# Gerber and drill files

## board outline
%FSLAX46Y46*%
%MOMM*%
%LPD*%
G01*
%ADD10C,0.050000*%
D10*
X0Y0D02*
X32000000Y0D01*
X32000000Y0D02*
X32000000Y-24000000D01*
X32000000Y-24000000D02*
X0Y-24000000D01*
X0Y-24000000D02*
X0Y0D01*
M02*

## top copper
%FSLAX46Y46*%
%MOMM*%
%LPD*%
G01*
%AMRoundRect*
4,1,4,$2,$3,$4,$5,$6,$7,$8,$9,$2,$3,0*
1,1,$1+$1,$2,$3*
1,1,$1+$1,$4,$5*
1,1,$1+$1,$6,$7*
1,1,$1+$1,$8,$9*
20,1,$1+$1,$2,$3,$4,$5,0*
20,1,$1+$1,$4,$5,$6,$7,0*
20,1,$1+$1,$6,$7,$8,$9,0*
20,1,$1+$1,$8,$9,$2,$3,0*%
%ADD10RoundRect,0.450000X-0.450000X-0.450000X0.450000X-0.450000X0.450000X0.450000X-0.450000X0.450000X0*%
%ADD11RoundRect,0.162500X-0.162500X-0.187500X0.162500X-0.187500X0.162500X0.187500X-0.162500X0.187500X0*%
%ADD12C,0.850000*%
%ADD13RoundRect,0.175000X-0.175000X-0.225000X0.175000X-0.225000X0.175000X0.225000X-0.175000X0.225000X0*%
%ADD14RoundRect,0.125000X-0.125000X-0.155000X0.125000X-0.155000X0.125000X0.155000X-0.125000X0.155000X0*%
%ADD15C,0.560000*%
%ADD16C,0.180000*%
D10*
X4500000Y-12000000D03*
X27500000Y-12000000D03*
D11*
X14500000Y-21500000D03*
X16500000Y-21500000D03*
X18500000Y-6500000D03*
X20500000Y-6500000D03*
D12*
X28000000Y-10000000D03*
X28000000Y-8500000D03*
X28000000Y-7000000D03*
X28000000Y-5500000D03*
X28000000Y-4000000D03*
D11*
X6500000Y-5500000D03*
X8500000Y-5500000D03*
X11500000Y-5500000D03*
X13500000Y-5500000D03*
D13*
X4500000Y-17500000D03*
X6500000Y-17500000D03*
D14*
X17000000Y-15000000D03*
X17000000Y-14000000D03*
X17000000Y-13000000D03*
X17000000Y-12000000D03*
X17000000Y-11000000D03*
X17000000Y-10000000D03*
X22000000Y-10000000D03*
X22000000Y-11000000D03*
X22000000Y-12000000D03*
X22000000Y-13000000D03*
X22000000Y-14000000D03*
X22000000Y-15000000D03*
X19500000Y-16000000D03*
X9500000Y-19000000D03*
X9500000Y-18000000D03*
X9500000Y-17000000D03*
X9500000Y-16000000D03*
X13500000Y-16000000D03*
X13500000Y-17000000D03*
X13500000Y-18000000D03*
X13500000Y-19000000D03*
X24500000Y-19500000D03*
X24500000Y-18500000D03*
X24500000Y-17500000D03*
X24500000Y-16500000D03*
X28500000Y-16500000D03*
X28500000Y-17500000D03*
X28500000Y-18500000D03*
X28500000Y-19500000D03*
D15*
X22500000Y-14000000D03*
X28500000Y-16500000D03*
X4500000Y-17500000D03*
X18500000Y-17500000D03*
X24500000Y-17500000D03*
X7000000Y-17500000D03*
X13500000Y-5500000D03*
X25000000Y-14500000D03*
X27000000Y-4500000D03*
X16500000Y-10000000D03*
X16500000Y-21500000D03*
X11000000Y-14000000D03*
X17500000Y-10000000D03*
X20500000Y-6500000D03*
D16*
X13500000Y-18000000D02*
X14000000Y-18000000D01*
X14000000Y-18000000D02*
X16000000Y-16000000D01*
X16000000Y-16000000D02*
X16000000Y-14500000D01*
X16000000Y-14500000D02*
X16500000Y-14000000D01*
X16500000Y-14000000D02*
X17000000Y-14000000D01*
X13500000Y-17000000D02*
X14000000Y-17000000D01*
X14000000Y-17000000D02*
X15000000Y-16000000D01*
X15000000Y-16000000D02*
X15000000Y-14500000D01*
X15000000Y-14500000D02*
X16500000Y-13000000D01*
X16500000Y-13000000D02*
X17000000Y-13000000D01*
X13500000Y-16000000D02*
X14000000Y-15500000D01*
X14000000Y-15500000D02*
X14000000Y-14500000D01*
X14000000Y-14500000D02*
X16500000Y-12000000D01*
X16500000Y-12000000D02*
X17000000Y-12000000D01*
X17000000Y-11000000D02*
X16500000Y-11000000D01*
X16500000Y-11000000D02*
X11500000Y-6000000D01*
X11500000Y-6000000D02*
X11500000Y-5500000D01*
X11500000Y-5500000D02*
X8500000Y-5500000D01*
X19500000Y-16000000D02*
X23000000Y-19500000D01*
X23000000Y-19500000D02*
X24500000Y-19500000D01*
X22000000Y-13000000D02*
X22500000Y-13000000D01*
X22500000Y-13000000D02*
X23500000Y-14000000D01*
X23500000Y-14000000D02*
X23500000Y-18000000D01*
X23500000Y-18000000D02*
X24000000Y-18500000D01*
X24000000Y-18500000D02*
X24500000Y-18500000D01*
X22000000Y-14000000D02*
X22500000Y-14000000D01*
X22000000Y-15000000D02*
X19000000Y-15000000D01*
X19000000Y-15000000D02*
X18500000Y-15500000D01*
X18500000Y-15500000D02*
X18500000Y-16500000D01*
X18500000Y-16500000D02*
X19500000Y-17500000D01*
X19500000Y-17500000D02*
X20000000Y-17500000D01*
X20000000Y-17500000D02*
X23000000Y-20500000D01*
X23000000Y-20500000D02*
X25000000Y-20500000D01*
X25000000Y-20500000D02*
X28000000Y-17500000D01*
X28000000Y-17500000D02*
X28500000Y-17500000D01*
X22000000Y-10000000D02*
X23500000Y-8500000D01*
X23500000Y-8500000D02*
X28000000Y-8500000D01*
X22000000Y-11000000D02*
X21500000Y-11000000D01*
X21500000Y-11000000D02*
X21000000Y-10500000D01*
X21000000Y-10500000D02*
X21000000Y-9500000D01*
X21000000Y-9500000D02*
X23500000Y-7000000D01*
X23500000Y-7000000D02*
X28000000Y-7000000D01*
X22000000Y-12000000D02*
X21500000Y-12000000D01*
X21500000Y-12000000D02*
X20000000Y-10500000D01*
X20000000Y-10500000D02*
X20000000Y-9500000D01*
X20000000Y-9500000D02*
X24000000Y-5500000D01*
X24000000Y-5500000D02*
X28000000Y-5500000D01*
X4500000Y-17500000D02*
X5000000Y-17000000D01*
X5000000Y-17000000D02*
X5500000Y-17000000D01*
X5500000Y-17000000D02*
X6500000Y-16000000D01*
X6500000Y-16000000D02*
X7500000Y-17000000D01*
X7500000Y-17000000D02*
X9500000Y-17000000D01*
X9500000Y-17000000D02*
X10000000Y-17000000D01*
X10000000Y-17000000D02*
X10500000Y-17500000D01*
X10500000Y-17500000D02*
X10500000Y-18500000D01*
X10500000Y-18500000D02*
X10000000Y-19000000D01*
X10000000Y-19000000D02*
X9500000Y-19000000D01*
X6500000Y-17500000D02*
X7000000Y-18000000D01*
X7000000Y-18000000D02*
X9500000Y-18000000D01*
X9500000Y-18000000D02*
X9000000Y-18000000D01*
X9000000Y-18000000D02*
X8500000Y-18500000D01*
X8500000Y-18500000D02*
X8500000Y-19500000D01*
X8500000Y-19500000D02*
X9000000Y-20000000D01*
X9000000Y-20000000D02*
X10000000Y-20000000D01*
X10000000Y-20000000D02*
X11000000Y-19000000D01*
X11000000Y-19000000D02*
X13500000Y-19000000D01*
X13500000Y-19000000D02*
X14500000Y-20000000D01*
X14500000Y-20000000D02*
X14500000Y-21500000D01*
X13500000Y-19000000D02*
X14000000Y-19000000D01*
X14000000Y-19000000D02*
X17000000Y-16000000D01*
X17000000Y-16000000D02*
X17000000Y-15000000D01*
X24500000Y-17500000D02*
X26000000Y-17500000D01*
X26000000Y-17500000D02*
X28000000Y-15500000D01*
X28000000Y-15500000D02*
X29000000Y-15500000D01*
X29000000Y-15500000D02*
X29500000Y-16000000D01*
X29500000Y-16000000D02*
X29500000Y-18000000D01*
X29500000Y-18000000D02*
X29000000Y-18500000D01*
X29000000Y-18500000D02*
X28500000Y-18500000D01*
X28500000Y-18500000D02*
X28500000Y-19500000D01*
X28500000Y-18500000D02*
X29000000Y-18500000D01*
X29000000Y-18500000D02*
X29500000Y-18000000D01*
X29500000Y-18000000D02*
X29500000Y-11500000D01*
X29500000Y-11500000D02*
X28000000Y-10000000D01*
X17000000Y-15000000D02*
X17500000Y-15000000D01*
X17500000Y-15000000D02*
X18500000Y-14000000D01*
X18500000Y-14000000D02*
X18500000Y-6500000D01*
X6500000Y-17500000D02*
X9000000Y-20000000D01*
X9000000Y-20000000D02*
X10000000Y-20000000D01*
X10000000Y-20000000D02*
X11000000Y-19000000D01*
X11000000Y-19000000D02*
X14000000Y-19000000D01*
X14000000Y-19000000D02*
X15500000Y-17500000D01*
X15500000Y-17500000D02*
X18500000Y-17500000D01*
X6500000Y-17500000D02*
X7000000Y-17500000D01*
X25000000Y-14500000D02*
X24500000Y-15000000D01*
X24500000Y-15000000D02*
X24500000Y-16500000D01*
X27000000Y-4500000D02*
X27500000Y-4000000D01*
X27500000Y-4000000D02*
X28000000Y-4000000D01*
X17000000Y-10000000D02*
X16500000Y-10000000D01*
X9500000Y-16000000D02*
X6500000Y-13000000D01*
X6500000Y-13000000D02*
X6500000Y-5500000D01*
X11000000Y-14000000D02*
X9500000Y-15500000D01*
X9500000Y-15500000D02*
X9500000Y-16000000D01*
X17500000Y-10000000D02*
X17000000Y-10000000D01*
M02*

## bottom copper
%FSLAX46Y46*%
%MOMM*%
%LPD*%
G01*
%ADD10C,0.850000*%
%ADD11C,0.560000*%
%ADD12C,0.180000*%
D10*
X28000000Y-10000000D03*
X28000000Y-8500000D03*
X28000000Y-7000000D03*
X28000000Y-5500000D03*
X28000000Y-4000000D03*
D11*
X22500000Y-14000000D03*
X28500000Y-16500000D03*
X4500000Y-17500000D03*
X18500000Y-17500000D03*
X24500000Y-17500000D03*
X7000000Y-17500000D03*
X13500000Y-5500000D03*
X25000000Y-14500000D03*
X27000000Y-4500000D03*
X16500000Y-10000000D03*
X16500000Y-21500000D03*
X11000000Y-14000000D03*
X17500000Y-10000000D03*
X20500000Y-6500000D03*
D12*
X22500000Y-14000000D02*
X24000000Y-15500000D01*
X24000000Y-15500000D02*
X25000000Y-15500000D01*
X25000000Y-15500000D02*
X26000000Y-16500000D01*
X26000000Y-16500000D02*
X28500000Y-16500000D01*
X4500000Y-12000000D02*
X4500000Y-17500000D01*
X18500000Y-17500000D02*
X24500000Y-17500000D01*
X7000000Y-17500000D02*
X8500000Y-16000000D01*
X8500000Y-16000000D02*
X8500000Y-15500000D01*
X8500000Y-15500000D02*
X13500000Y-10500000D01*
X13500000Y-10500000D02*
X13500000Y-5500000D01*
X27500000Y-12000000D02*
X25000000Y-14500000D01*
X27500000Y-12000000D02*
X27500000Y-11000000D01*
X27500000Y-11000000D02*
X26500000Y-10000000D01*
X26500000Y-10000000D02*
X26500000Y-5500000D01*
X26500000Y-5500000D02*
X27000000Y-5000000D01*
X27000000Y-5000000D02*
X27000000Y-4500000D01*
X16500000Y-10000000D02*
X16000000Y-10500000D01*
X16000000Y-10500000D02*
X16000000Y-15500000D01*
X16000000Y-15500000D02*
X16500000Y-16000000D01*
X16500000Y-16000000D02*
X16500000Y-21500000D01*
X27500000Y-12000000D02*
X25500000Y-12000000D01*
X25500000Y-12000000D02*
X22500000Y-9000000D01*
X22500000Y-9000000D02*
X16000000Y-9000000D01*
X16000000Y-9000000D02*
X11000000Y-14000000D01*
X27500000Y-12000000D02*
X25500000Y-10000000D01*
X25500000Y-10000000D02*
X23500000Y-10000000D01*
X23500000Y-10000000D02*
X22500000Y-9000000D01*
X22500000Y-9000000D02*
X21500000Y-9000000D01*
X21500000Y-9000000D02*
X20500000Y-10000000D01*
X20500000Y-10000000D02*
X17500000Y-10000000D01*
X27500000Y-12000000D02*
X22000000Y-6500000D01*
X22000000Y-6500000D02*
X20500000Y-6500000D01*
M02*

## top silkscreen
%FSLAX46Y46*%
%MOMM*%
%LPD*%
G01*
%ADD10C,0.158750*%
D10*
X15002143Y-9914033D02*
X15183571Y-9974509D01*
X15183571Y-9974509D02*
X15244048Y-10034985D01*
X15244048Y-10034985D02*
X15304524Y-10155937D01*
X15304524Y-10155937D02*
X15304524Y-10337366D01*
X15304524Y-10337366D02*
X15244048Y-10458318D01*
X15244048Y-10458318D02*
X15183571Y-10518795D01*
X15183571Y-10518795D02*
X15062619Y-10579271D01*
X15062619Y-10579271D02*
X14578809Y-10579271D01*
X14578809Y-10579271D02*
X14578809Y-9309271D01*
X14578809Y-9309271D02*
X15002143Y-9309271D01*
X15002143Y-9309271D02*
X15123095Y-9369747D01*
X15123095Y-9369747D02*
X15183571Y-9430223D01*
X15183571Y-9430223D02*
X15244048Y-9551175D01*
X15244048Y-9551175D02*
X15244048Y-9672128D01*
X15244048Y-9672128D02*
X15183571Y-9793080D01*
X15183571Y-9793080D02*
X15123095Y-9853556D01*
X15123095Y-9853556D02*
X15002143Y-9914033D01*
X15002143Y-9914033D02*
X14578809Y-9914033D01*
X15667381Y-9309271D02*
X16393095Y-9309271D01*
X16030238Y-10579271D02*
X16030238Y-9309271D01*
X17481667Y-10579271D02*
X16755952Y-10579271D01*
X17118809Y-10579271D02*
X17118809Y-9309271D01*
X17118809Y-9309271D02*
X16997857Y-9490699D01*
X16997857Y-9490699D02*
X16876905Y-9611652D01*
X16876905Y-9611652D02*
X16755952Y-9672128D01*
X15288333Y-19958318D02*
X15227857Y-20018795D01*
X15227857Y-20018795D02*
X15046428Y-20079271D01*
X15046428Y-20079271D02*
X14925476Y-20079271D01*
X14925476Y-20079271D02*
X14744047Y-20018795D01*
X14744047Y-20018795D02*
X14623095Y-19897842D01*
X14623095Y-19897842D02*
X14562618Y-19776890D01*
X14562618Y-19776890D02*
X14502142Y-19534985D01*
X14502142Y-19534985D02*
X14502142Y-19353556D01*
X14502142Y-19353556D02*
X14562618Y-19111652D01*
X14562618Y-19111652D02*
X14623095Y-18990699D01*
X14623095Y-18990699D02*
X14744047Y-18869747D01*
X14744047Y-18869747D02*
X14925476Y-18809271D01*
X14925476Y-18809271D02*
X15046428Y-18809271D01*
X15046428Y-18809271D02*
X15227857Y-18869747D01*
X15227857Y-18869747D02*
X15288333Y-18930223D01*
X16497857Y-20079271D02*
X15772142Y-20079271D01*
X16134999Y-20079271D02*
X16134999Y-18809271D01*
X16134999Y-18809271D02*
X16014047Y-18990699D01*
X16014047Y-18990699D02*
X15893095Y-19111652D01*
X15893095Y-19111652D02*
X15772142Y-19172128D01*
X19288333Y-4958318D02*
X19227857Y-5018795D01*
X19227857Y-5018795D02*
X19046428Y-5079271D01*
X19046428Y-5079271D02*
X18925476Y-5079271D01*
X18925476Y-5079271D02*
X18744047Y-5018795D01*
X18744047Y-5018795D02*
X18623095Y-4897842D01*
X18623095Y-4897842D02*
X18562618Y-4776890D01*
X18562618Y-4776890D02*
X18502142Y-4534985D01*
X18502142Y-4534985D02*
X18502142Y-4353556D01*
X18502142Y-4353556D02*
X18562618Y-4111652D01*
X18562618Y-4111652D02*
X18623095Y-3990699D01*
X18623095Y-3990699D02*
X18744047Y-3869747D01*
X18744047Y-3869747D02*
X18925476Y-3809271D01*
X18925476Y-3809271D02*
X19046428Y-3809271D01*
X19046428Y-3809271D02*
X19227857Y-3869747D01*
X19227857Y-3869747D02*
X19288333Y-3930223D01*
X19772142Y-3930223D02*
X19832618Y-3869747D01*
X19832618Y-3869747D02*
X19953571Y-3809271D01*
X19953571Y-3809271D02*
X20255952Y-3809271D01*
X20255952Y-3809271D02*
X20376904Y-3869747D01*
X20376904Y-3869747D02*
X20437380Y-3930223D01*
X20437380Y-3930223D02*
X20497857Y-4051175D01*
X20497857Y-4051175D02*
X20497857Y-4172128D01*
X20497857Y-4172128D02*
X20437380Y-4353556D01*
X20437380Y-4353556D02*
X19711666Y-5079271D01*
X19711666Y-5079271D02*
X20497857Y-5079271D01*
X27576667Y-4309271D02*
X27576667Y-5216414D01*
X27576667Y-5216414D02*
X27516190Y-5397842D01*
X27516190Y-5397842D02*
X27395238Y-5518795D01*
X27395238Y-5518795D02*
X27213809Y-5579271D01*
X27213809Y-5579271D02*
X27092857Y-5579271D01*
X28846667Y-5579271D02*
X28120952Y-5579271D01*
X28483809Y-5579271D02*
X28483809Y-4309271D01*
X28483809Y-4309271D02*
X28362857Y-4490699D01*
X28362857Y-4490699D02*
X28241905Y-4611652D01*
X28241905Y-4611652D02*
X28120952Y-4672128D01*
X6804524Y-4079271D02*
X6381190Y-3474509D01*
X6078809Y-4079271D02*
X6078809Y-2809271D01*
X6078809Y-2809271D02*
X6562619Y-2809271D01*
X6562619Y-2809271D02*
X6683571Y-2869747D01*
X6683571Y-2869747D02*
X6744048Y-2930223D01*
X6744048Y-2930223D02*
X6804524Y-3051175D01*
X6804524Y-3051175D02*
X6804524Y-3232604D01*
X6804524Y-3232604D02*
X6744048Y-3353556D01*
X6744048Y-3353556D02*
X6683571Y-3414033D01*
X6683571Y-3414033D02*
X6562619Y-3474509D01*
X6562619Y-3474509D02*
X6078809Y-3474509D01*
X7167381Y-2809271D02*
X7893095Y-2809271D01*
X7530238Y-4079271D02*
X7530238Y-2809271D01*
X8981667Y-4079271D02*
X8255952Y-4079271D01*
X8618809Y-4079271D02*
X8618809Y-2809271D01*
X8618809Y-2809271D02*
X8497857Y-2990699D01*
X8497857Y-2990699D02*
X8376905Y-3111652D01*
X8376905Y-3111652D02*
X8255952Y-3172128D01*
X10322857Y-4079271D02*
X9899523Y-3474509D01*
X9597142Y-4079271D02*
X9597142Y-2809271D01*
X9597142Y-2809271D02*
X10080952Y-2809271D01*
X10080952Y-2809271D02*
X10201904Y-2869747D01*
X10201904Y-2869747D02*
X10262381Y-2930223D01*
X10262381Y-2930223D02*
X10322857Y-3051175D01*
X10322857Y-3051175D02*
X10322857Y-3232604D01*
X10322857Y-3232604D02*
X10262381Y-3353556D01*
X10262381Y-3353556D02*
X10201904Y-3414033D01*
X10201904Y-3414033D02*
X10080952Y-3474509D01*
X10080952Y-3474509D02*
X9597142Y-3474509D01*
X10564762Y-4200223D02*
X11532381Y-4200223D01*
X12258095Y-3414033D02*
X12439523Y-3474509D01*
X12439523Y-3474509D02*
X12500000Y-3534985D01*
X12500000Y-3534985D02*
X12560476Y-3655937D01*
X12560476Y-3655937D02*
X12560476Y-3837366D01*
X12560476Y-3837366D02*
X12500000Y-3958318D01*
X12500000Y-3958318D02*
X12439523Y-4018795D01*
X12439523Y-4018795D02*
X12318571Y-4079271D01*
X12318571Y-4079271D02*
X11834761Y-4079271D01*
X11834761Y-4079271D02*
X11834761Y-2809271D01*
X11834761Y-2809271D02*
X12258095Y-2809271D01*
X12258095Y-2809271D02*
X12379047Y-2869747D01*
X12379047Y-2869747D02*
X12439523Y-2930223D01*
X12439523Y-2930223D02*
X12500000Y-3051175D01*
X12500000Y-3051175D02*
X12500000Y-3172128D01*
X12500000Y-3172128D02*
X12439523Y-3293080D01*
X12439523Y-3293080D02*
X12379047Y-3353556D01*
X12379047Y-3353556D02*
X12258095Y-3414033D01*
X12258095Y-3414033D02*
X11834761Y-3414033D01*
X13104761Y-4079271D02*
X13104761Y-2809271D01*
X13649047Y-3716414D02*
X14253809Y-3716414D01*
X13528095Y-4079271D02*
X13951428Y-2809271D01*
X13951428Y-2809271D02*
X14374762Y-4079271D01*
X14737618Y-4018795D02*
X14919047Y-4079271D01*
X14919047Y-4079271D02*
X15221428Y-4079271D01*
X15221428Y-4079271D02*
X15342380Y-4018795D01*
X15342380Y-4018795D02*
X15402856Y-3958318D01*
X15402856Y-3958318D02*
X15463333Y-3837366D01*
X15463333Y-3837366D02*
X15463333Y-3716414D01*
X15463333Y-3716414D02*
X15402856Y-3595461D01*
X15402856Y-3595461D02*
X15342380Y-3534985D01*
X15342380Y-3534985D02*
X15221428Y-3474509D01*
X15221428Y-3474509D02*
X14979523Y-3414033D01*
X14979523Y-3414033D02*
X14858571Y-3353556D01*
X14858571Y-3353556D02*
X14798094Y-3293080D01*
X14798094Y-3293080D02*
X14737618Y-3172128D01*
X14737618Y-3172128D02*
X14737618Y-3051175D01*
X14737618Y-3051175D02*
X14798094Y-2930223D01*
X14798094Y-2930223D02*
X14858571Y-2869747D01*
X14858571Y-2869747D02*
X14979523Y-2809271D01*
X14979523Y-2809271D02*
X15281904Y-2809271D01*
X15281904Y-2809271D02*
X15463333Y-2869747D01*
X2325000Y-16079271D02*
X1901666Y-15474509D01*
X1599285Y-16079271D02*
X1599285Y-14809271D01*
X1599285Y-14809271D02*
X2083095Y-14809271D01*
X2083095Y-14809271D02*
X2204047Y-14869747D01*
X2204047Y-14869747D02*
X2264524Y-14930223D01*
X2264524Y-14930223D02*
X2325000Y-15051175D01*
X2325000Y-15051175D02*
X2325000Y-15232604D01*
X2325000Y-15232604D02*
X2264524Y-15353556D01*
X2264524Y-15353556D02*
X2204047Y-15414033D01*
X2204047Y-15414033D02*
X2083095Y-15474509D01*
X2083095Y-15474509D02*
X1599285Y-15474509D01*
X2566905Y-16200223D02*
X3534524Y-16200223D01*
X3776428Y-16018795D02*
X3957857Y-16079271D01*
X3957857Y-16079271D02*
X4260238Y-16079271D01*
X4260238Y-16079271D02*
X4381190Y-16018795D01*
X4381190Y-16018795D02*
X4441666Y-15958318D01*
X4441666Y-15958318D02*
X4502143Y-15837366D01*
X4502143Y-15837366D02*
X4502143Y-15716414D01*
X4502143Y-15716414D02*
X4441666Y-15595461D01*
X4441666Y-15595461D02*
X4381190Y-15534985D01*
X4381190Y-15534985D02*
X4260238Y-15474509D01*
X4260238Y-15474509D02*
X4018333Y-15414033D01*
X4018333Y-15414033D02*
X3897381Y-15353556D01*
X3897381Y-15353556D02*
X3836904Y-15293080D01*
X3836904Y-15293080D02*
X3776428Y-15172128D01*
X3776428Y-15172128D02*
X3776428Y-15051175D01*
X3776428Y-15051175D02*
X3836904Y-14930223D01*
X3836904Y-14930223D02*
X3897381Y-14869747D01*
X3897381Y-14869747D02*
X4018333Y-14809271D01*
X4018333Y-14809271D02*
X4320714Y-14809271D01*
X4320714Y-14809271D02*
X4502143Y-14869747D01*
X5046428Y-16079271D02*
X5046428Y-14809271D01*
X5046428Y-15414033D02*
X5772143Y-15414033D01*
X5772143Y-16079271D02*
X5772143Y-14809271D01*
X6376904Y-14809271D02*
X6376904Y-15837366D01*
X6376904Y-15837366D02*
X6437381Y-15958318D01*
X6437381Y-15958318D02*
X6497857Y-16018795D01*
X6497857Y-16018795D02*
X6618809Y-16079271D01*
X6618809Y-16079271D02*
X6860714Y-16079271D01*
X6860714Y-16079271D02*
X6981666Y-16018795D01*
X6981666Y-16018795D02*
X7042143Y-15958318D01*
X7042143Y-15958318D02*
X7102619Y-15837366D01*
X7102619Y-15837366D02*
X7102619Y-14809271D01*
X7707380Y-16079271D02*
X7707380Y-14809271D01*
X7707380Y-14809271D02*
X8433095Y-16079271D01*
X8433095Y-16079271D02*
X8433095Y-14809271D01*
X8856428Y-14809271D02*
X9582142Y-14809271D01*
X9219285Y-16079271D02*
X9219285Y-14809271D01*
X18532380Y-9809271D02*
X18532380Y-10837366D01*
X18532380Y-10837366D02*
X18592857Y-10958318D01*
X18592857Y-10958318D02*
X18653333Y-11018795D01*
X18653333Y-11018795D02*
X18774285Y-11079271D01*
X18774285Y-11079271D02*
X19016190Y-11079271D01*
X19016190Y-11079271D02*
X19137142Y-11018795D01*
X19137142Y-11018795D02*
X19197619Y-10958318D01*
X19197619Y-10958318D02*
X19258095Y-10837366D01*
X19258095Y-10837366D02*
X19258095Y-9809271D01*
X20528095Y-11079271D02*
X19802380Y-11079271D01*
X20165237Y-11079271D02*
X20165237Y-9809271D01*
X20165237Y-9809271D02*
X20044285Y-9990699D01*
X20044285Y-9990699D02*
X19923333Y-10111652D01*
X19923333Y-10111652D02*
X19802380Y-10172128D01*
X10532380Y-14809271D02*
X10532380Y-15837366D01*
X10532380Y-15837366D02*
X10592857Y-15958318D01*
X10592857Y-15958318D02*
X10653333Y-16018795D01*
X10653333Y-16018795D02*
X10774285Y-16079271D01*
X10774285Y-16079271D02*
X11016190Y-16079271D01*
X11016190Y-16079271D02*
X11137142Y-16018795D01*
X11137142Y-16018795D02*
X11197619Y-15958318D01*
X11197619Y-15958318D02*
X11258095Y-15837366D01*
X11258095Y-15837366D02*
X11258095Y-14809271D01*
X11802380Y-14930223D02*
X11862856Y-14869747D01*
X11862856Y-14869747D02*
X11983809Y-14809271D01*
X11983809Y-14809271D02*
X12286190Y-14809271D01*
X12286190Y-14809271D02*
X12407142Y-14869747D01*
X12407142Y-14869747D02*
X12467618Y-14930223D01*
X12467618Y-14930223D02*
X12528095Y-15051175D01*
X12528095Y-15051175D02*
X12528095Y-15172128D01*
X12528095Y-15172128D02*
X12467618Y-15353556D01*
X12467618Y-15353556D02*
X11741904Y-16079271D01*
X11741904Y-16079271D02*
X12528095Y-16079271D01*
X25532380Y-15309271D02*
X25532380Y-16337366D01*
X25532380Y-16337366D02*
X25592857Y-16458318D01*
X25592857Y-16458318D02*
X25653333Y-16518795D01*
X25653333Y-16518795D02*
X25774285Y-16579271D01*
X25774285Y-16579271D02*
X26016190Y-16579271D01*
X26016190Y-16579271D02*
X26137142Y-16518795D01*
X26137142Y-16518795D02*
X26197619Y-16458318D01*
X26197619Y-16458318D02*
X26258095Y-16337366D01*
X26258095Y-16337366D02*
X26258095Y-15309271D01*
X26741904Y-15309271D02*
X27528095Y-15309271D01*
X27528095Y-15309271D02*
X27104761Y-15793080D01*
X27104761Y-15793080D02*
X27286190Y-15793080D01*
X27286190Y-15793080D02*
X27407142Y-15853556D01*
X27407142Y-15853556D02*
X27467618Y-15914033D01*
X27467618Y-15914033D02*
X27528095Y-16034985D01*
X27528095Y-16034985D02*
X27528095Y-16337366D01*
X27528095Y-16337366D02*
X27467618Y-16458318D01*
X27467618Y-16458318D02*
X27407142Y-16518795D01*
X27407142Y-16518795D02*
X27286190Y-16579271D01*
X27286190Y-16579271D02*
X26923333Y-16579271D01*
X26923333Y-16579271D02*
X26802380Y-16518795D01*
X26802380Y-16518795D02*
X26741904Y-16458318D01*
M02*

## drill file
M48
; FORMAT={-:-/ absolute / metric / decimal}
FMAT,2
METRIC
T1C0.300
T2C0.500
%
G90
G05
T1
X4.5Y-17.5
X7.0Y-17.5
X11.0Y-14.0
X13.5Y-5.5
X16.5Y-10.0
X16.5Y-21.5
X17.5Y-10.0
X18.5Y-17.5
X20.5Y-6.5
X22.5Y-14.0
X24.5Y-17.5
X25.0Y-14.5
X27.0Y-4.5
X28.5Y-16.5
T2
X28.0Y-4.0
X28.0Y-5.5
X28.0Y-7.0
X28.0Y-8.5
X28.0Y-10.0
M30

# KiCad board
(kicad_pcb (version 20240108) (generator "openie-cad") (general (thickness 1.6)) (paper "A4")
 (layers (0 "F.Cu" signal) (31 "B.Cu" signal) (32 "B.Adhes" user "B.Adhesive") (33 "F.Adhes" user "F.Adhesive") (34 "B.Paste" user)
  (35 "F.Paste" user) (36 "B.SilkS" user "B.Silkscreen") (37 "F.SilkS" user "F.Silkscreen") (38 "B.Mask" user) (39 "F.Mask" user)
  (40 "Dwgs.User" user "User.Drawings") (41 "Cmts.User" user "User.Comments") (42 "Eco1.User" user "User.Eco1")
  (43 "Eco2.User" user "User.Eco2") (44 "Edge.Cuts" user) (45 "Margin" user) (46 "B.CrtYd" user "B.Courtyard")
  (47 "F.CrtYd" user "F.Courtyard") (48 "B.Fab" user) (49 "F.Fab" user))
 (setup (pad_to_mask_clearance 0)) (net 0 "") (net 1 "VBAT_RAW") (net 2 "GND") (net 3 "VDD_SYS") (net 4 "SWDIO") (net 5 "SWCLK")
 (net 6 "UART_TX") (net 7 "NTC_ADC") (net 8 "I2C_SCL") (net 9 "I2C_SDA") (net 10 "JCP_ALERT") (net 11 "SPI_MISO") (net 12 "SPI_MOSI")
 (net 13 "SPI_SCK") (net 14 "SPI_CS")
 (gr_line (start 0.0000 0.0000) (end 32.0000 0.0000) (layer "Edge.Cuts") (width 0.05))
 (gr_line (start 32.0000 0.0000) (end 32.0000 24.0000) (layer "Edge.Cuts") (width 0.05))
 (gr_line (start 32.0000 24.0000) (end 0.0000 24.0000) (layer "Edge.Cuts") (width 0.05))
 (gr_line (start 0.0000 24.0000) (end 0.0000 0.0000) (layer "Edge.Cuts") (width 0.05))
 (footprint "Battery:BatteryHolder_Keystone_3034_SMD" (layer "B.Cu") (at 16.0000 12.0000 0.00)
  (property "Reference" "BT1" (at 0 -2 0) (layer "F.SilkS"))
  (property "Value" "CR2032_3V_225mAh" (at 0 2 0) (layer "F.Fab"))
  (pad "1" smd roundrect (at -11.5000 0.0000) (size 1.8000 1.8000) (layers "F.Cu" "F.Paste" "F.Mask") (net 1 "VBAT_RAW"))
  (pad "2" smd roundrect (at 11.5000 0.0000) (size 1.8000 1.8000) (layers "F.Cu" "F.Paste" "F.Mask") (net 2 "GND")))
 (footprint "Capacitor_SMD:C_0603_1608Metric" (layer "F.Cu") (at 15.5000 21.5000 0.00)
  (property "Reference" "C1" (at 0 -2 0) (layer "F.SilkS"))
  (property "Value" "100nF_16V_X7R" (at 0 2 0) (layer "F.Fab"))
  (pad "1" smd roundrect (at -1.0000 0.0000) (size 0.6500 0.7000) (layers "F.Cu" "F.Paste" "F.Mask") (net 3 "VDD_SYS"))
  (pad "2" smd roundrect (at 1.0000 0.0000) (size 0.6500 0.7000) (layers "F.Cu" "F.Paste" "F.Mask") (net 2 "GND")))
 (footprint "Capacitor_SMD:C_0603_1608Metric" (layer "F.Cu") (at 19.5000 6.5000 0.00)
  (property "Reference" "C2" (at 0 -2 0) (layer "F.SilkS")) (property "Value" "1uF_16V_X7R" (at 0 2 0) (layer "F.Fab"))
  (pad "1" smd roundrect (at -1.0000 0.0000) (size 0.6500 0.7000) (layers "F.Cu" "F.Paste" "F.Mask") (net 3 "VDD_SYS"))
  (pad "2" smd roundrect (at 1.0000 0.0000) (size 0.6500 0.7000) (layers "F.Cu" "F.Paste" "F.Mask") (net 2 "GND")))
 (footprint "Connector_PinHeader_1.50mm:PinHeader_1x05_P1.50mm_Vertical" (layer "F.Cu") (at 28.0000 7.0000 0.00)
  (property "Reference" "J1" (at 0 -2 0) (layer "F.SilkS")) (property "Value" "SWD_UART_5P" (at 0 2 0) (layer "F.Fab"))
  (pad "1" thru_hole circle (at 0.0000 3.0000) (size 0.8500 0.8500) (layers "*.Cu" "*.Mask") (drill 0.5000) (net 3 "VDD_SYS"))
  (pad "2" thru_hole circle (at 0.0000 1.5000) (size 0.8500 0.8500) (layers "*.Cu" "*.Mask") (drill 0.5000) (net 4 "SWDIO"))
  (pad "3" thru_hole circle (at 0.0000 0.0000) (size 0.8500 0.8500) (layers "*.Cu" "*.Mask") (drill 0.5000) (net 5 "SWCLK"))
  (pad "4" thru_hole circle (at 0.0000 -1.5000) (size 0.8500 0.8500) (layers "*.Cu" "*.Mask") (drill 0.5000) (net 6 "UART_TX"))
  (pad "5" thru_hole circle (at 0.0000 -3.0000) (size 0.8500 0.8500) (layers "*.Cu" "*.Mask") (drill 0.5000) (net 2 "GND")))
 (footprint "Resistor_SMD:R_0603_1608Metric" (layer "F.Cu") (at 7.5000 5.5000 0.00)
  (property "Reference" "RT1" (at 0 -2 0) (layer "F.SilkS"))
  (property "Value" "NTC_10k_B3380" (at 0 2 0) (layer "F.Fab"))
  (pad "1" smd roundrect (at -1.0000 0.0000) (size 0.6500 0.7000) (layers "F.Cu" "F.Paste" "F.Mask") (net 2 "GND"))
  (pad "2" smd roundrect (at 1.0000 0.0000) (size 0.6500 0.7000) (layers "F.Cu" "F.Paste" "F.Mask") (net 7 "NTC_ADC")))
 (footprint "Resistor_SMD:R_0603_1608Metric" (layer "F.Cu") (at 12.5000 5.5000 0.00)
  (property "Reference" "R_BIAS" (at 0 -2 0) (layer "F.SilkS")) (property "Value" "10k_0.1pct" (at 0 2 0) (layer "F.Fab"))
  (pad "1" smd roundrect (at -1.0000 0.0000) (size 0.6500 0.7000) (layers "F.Cu" "F.Paste" "F.Mask") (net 7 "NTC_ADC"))
  (pad "2" smd roundrect (at 1.0000 0.0000) (size 0.6500 0.7000) (layers "F.Cu" "F.Paste" "F.Mask") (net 3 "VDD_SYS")))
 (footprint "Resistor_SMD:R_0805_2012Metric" (layer "F.Cu") (at 5.5000 17.5000 0.00)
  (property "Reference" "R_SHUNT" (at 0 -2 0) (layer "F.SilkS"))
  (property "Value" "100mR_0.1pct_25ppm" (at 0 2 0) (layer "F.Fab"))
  (pad "1" smd roundrect (at -1.0000 0.0000) (size 0.7000 0.8000) (layers "F.Cu" "F.Paste" "F.Mask") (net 1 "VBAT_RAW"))
  (pad "2" smd roundrect (at 1.0000 0.0000) (size 0.7000 0.8000) (layers "F.Cu" "F.Paste" "F.Mask") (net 3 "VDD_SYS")))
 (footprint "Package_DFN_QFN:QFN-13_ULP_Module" (layer "F.Cu") (at 19.5000 12.5000 0.00)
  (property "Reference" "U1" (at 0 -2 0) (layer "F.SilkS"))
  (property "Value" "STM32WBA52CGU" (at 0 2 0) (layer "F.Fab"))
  (pad "1" smd roundrect (at -2.5000 2.5000) (size 0.5000 0.5600) (layers "F.Cu" "F.Paste" "F.Mask") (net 3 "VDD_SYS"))
  (pad "2" smd roundrect (at -2.5000 1.5000) (size 0.5000 0.5600) (layers "F.Cu" "F.Paste" "F.Mask") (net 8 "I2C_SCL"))
  (pad "3" smd roundrect (at -2.5000 0.5000) (size 0.5000 0.5600) (layers "F.Cu" "F.Paste" "F.Mask") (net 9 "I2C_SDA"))
  (pad "4" smd roundrect (at -2.5000 -0.5000) (size 0.5000 0.5600) (layers "F.Cu" "F.Paste" "F.Mask") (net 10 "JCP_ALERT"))
  (pad "5" smd roundrect (at -2.5000 -1.5000) (size 0.5000 0.5600) (layers "F.Cu" "F.Paste" "F.Mask") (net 7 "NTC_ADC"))
  (pad "6" smd roundrect (at -2.5000 -2.5000) (size 0.5000 0.5600) (layers "F.Cu" "F.Paste" "F.Mask") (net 2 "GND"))
  (pad "7" smd roundrect (at 2.5000 -2.5000) (size 0.5000 0.5600) (layers "F.Cu" "F.Paste" "F.Mask") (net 4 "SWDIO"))
  (pad "8" smd roundrect (at 2.5000 -1.5000) (size 0.5000 0.5600) (layers "F.Cu" "F.Paste" "F.Mask") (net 5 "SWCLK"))
  (pad "9" smd roundrect (at 2.5000 -0.5000) (size 0.5000 0.5600) (layers "F.Cu" "F.Paste" "F.Mask") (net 6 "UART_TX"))
  (pad "10" smd roundrect (at 2.5000 0.5000) (size 0.5000 0.5600) (layers "F.Cu" "F.Paste" "F.Mask") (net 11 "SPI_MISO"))
  (pad "11" smd roundrect (at 2.5000 1.5000) (size 0.5000 0.5600) (layers "F.Cu" "F.Paste" "F.Mask") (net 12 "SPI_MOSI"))
  (pad "12" smd roundrect (at 2.5000 2.5000) (size 0.5000 0.5600) (layers "F.Cu" "F.Paste" "F.Mask") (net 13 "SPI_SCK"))
  (pad "13" smd roundrect (at 0.0000 3.5000) (size 0.5000 0.5600) (layers "F.Cu" "F.Paste" "F.Mask") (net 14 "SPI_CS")))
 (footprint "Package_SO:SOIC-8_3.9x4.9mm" (layer "F.Cu") (at 11.5000 17.5000 0.00) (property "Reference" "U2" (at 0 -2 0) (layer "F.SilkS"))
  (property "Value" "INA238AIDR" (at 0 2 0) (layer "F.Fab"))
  (pad "1" smd roundrect (at -2.0000 1.5000) (size 0.5000 0.5600) (layers "F.Cu" "F.Paste" "F.Mask") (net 1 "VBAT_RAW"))
  (pad "2" smd roundrect (at -2.0000 0.5000) (size 0.5000 0.5600) (layers "F.Cu" "F.Paste" "F.Mask") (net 3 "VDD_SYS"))
  (pad "3" smd roundrect (at -2.0000 -0.5000) (size 0.5000 0.5600) (layers "F.Cu" "F.Paste" "F.Mask") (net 1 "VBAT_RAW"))
  (pad "4" smd roundrect (at -2.0000 -1.5000) (size 0.5000 0.5600) (layers "F.Cu" "F.Paste" "F.Mask") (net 2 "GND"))
  (pad "5" smd roundrect (at 2.0000 -1.5000) (size 0.5000 0.5600) (layers "F.Cu" "F.Paste" "F.Mask") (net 10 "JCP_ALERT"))
  (pad "6" smd roundrect (at 2.0000 -0.5000) (size 0.5000 0.5600) (layers "F.Cu" "F.Paste" "F.Mask") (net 9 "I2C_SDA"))
  (pad "7" smd roundrect (at 2.0000 0.5000) (size 0.5000 0.5600) (layers "F.Cu" "F.Paste" "F.Mask") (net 8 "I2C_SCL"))
  (pad "8" smd roundrect (at 2.0000 1.5000) (size 0.5000 0.5600) (layers "F.Cu" "F.Paste" "F.Mask") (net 3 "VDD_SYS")))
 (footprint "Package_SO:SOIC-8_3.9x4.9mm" (layer "F.Cu") (at 26.5000 18.0000 0.00) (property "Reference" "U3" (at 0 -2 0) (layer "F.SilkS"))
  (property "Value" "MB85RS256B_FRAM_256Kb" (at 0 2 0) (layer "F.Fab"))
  (pad "1" smd roundrect (at -2.0000 1.5000) (size 0.5000 0.5600) (layers "F.Cu" "F.Paste" "F.Mask") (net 14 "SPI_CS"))
  (pad "2" smd roundrect (at -2.0000 0.5000) (size 0.5000 0.5600) (layers "F.Cu" "F.Paste" "F.Mask") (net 11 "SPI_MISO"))
  (pad "3" smd roundrect (at -2.0000 -0.5000) (size 0.5000 0.5600) (layers "F.Cu" "F.Paste" "F.Mask") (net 3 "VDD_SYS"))
  (pad "4" smd roundrect (at -2.0000 -1.5000) (size 0.5000 0.5600) (layers "F.Cu" "F.Paste" "F.Mask") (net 2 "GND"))
  (pad "5" smd roundrect (at 2.0000 -1.5000) (size 0.5000 0.5600) (layers "F.Cu" "F.Paste" "F.Mask") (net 12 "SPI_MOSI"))
  (pad "6" smd roundrect (at 2.0000 -0.5000) (size 0.5000 0.5600) (layers "F.Cu" "F.Paste" "F.Mask") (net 13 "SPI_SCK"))
  (pad "7" smd roundrect (at 2.0000 0.5000) (size 0.5000 0.5600) (layers "F.Cu" "F.Paste" "F.Mask") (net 3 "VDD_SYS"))
  (pad "8" smd roundrect (at 2.0000 1.5000) (size 0.5000 0.5600) (layers "F.Cu" "F.Paste" "F.Mask") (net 3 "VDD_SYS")))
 (segment (start 13.5000 18.0000) (end 14.0000 18.0000) (width 0.180) (layer "F.Cu") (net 8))
 (segment (start 14.0000 18.0000) (end 16.0000 16.0000) (width 0.180) (layer "F.Cu") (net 8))
 (segment (start 16.0000 16.0000) (end 16.0000 14.5000) (width 0.180) (layer "F.Cu") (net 8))
 (segment (start 16.0000 14.5000) (end 16.5000 14.0000) (width 0.180) (layer "F.Cu") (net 8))
 (segment (start 16.5000 14.0000) (end 17.0000 14.0000) (width 0.180) (layer "F.Cu") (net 8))
 (segment (start 13.5000 17.0000) (end 14.0000 17.0000) (width 0.180) (layer "F.Cu") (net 9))
 (segment (start 14.0000 17.0000) (end 15.0000 16.0000) (width 0.180) (layer "F.Cu") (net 9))
 (segment (start 15.0000 16.0000) (end 15.0000 14.5000) (width 0.180) (layer "F.Cu") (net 9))
 (segment (start 15.0000 14.5000) (end 16.5000 13.0000) (width 0.180) (layer "F.Cu") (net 9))
 (segment (start 16.5000 13.0000) (end 17.0000 13.0000) (width 0.180) (layer "F.Cu") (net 9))
 (segment (start 13.5000 16.0000) (end 14.0000 15.5000) (width 0.180) (layer "F.Cu") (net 10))
 (segment (start 14.0000 15.5000) (end 14.0000 14.5000) (width 0.180) (layer "F.Cu") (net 10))
 (segment (start 14.0000 14.5000) (end 16.5000 12.0000) (width 0.180) (layer "F.Cu") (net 10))
 (segment (start 16.5000 12.0000) (end 17.0000 12.0000) (width 0.180) (layer "F.Cu") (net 10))
 (segment (start 17.0000 11.0000) (end 16.5000 11.0000) (width 0.180) (layer "F.Cu") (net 7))
 (segment (start 16.5000 11.0000) (end 11.5000 6.0000) (width 0.180) (layer "F.Cu") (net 7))
 (segment (start 11.5000 6.0000) (end 11.5000 5.5000) (width 0.180) (layer "F.Cu") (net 7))
 (segment (start 11.5000 5.5000) (end 8.5000 5.5000) (width 0.180) (layer "F.Cu") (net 7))
 (segment (start 19.5000 16.0000) (end 23.0000 19.5000) (width 0.180) (layer "F.Cu") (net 14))
 (segment (start 23.0000 19.5000) (end 24.5000 19.5000) (width 0.180) (layer "F.Cu") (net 14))
 (segment (start 22.0000 13.0000) (end 22.5000 13.0000) (width 0.180) (layer "F.Cu") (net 11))
 (segment (start 22.5000 13.0000) (end 23.5000 14.0000) (width 0.180) (layer "F.Cu") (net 11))
 (segment (start 23.5000 14.0000) (end 23.5000 18.0000) (width 0.180) (layer "F.Cu") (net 11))
 (segment (start 23.5000 18.0000) (end 24.0000 18.5000) (width 0.180) (layer "F.Cu") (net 11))
 (segment (start 24.0000 18.5000) (end 24.5000 18.5000) (width 0.180) (layer "F.Cu") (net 11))
 (segment (start 22.0000 14.0000) (end 22.5000 14.0000) (width 0.180) (layer "F.Cu") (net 12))
 (segment (start 22.5000 14.0000) (end 24.0000 15.5000) (width 0.180) (layer "B.Cu") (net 12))
 (segment (start 24.0000 15.5000) (end 25.0000 15.5000) (width 0.180) (layer "B.Cu") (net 12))
 (segment (start 25.0000 15.5000) (end 26.0000 16.5000) (width 0.180) (layer "B.Cu") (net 12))
 (segment (start 26.0000 16.5000) (end 28.5000 16.5000) (width 0.180) (layer "B.Cu") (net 12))
 (segment (start 22.0000 15.0000) (end 19.0000 15.0000) (width 0.180) (layer "F.Cu") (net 13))
 (segment (start 19.0000 15.0000) (end 18.5000 15.5000) (width 0.180) (layer "F.Cu") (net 13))
 (segment (start 18.5000 15.5000) (end 18.5000 16.5000) (width 0.180) (layer "F.Cu") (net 13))
 (segment (start 18.5000 16.5000) (end 19.5000 17.5000) (width 0.180) (layer "F.Cu") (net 13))
 (segment (start 19.5000 17.5000) (end 20.0000 17.5000) (width 0.180) (layer "F.Cu") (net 13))
 (segment (start 20.0000 17.5000) (end 23.0000 20.5000) (width 0.180) (layer "F.Cu") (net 13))
 (segment (start 23.0000 20.5000) (end 25.0000 20.5000) (width 0.180) (layer "F.Cu") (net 13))
 (segment (start 25.0000 20.5000) (end 28.0000 17.5000) (width 0.180) (layer "F.Cu") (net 13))
 (segment (start 28.0000 17.5000) (end 28.5000 17.5000) (width 0.180) (layer "F.Cu") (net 13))
 (segment (start 22.0000 10.0000) (end 23.5000 8.5000) (width 0.180) (layer "F.Cu") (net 4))
 (segment (start 23.5000 8.5000) (end 28.0000 8.5000) (width 0.180) (layer "F.Cu") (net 4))
 (segment (start 22.0000 11.0000) (end 21.5000 11.0000) (width 0.180) (layer "F.Cu") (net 5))
 (segment (start 21.5000 11.0000) (end 21.0000 10.5000) (width 0.180) (layer "F.Cu") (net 5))
 (segment (start 21.0000 10.5000) (end 21.0000 9.5000) (width 0.180) (layer "F.Cu") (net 5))
 (segment (start 21.0000 9.5000) (end 23.5000 7.0000) (width 0.180) (layer "F.Cu") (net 5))
 (segment (start 23.5000 7.0000) (end 28.0000 7.0000) (width 0.180) (layer "F.Cu") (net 5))
 (segment (start 22.0000 12.0000) (end 21.5000 12.0000) (width 0.180) (layer "F.Cu") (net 6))
 (segment (start 21.5000 12.0000) (end 20.0000 10.5000) (width 0.180) (layer "F.Cu") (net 6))
 (segment (start 20.0000 10.5000) (end 20.0000 9.5000) (width 0.180) (layer "F.Cu") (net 6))
 (segment (start 20.0000 9.5000) (end 24.0000 5.5000) (width 0.180) (layer "F.Cu") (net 6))
 (segment (start 24.0000 5.5000) (end 28.0000 5.5000) (width 0.180) (layer "F.Cu") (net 6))
 (segment (start 4.5000 12.0000) (end 4.5000 17.5000) (width 0.180) (layer "B.Cu") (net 1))
 (segment (start 4.5000 17.5000) (end 5.0000 17.0000) (width 0.180) (layer "F.Cu") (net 1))
 (segment (start 5.0000 17.0000) (end 5.5000 17.0000) (width 0.180) (layer "F.Cu") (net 1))
 (segment (start 5.5000 17.0000) (end 6.5000 16.0000) (width 0.180) (layer "F.Cu") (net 1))
 (segment (start 6.5000 16.0000) (end 7.5000 17.0000) (width 0.180) (layer "F.Cu") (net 1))
 (segment (start 7.5000 17.0000) (end 9.5000 17.0000) (width 0.180) (layer "F.Cu") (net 1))
 (segment (start 9.5000 17.0000) (end 10.0000 17.0000) (width 0.180) (layer "F.Cu") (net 1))
 (segment (start 10.0000 17.0000) (end 10.5000 17.5000) (width 0.180) (layer "F.Cu") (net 1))
 (segment (start 10.5000 17.5000) (end 10.5000 18.5000) (width 0.180) (layer "F.Cu") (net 1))
 (segment (start 10.5000 18.5000) (end 10.0000 19.0000) (width 0.180) (layer "F.Cu") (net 1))
 (segment (start 10.0000 19.0000) (end 9.5000 19.0000) (width 0.180) (layer "F.Cu") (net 1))
 (segment (start 6.5000 17.5000) (end 7.0000 18.0000) (width 0.180) (layer "F.Cu") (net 3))
 (segment (start 7.0000 18.0000) (end 9.5000 18.0000) (width 0.180) (layer "F.Cu") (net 3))
 (segment (start 9.5000 18.0000) (end 9.0000 18.0000) (width 0.180) (layer "F.Cu") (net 3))
 (segment (start 9.0000 18.0000) (end 8.5000 18.5000) (width 0.180) (layer "F.Cu") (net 3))
 (segment (start 8.5000 18.5000) (end 8.5000 19.5000) (width 0.180) (layer "F.Cu") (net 3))
 (segment (start 8.5000 19.5000) (end 9.0000 20.0000) (width 0.180) (layer "F.Cu") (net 3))
 (segment (start 9.0000 20.0000) (end 10.0000 20.0000) (width 0.180) (layer "F.Cu") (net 3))
 (segment (start 10.0000 20.0000) (end 11.0000 19.0000) (width 0.180) (layer "F.Cu") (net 3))
 (segment (start 11.0000 19.0000) (end 13.5000 19.0000) (width 0.180) (layer "F.Cu") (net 3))
 (segment (start 13.5000 19.0000) (end 14.5000 20.0000) (width 0.180) (layer "F.Cu") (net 3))
 (segment (start 14.5000 20.0000) (end 14.5000 21.5000) (width 0.180) (layer "F.Cu") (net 3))
 (segment (start 13.5000 19.0000) (end 14.0000 19.0000) (width 0.180) (layer "F.Cu") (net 3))
 (segment (start 14.0000 19.0000) (end 17.0000 16.0000) (width 0.180) (layer "F.Cu") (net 3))
 (segment (start 17.0000 16.0000) (end 17.0000 15.0000) (width 0.180) (layer "F.Cu") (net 3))
 (segment (start 24.5000 17.5000) (end 26.0000 17.5000) (width 0.180) (layer "F.Cu") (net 3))
 (segment (start 26.0000 17.5000) (end 28.0000 15.5000) (width 0.180) (layer "F.Cu") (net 3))
 (segment (start 28.0000 15.5000) (end 29.0000 15.5000) (width 0.180) (layer "F.Cu") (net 3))
 (segment (start 29.0000 15.5000) (end 29.5000 16.0000) (width 0.180) (layer "F.Cu") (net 3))
 (segment (start 29.5000 16.0000) (end 29.5000 18.0000) (width 0.180) (layer "F.Cu") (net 3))
 (segment (start 29.5000 18.0000) (end 29.0000 18.5000) (width 0.180) (layer "F.Cu") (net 3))
 (segment (start 29.0000 18.5000) (end 28.5000 18.5000) (width 0.180) (layer "F.Cu") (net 3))
 (segment (start 28.5000 18.5000) (end 28.5000 19.5000) (width 0.180) (layer "F.Cu") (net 3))
 (segment (start 28.5000 18.5000) (end 29.0000 18.5000) (width 0.180) (layer "F.Cu") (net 3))
 (segment (start 29.0000 18.5000) (end 29.5000 18.0000) (width 0.180) (layer "F.Cu") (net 3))
 (segment (start 29.5000 18.0000) (end 29.5000 11.5000) (width 0.180) (layer "F.Cu") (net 3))
 (segment (start 29.5000 11.5000) (end 28.0000 10.0000) (width 0.180) (layer "F.Cu") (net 3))
 (segment (start 17.0000 15.0000) (end 17.5000 15.0000) (width 0.180) (layer "F.Cu") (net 3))
 (segment (start 17.5000 15.0000) (end 18.5000 14.0000) (width 0.180) (layer "F.Cu") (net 3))
 (segment (start 18.5000 14.0000) (end 18.5000 6.5000) (width 0.180) (layer "F.Cu") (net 3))
 (segment (start 6.5000 17.5000) (end 9.0000 20.0000) (width 0.180) (layer "F.Cu") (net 3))
 (segment (start 9.0000 20.0000) (end 10.0000 20.0000) (width 0.180) (layer "F.Cu") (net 3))
 (segment (start 10.0000 20.0000) (end 11.0000 19.0000) (width 0.180) (layer "F.Cu") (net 3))
 (segment (start 11.0000 19.0000) (end 14.0000 19.0000) (width 0.180) (layer "F.Cu") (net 3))
 (segment (start 14.0000 19.0000) (end 15.5000 17.5000) (width 0.180) (layer "F.Cu") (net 3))
 (segment (start 15.5000 17.5000) (end 18.5000 17.5000) (width 0.180) (layer "F.Cu") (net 3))
 (segment (start 18.5000 17.5000) (end 24.5000 17.5000) (width 0.180) (layer "B.Cu") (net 3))
 (segment (start 6.5000 17.5000) (end 7.0000 17.5000) (width 0.180) (layer "F.Cu") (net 3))
 (segment (start 7.0000 17.5000) (end 8.5000 16.0000) (width 0.180) (layer "B.Cu") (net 3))
 (segment (start 8.5000 16.0000) (end 8.5000 15.5000) (width 0.180) (layer "B.Cu") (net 3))
 (segment (start 8.5000 15.5000) (end 13.5000 10.5000) (width 0.180) (layer "B.Cu") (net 3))
 (segment (start 13.5000 10.5000) (end 13.5000 5.5000) (width 0.180) (layer "B.Cu") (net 3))
 (segment (start 27.5000 12.0000) (end 25.0000 14.5000) (width 0.180) (layer "B.Cu") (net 2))
 (segment (start 25.0000 14.5000) (end 24.5000 15.0000) (width 0.180) (layer "F.Cu") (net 2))
 (segment (start 24.5000 15.0000) (end 24.5000 16.5000) (width 0.180) (layer "F.Cu") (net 2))
 (segment (start 27.5000 12.0000) (end 27.5000 11.0000) (width 0.180) (layer "B.Cu") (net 2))
 (segment (start 27.5000 11.0000) (end 26.5000 10.0000) (width 0.180) (layer "B.Cu") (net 2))
 (segment (start 26.5000 10.0000) (end 26.5000 5.5000) (width 0.180) (layer "B.Cu") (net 2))
 (segment (start 26.5000 5.5000) (end 27.0000 5.0000) (width 0.180) (layer "B.Cu") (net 2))
 (segment (start 27.0000 5.0000) (end 27.0000 4.5000) (width 0.180) (layer "B.Cu") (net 2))
 (segment (start 27.0000 4.5000) (end 27.5000 4.0000) (width 0.180) (layer "F.Cu") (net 2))
 (segment (start 27.5000 4.0000) (end 28.0000 4.0000) (width 0.180) (layer "F.Cu") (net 2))
 (segment (start 17.0000 10.0000) (end 16.5000 10.0000) (width 0.180) (layer "F.Cu") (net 2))
 (segment (start 16.5000 10.0000) (end 16.0000 10.5000) (width 0.180) (layer "B.Cu") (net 2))
 (segment (start 16.0000 10.5000) (end 16.0000 15.5000) (width 0.180) (layer "B.Cu") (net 2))
 (segment (start 16.0000 15.5000) (end 16.5000 16.0000) (width 0.180) (layer "B.Cu") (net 2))
 (segment (start 16.5000 16.0000) (end 16.5000 21.5000) (width 0.180) (layer "B.Cu") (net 2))
 (segment (start 9.5000 16.0000) (end 6.5000 13.0000) (width 0.180) (layer "F.Cu") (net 2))
 (segment (start 6.5000 13.0000) (end 6.5000 5.5000) (width 0.180) (layer "F.Cu") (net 2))
 (segment (start 27.5000 12.0000) (end 25.5000 12.0000) (width 0.180) (layer "B.Cu") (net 2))
 (segment (start 25.5000 12.0000) (end 22.5000 9.0000) (width 0.180) (layer "B.Cu") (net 2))
 (segment (start 22.5000 9.0000) (end 16.0000 9.0000) (width 0.180) (layer "B.Cu") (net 2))
 (segment (start 16.0000 9.0000) (end 11.0000 14.0000) (width 0.180) (layer "B.Cu") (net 2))
 (segment (start 11.0000 14.0000) (end 9.5000 15.5000) (width 0.180) (layer "F.Cu") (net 2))
 (segment (start 9.5000 15.5000) (end 9.5000 16.0000) (width 0.180) (layer "F.Cu") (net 2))
 (segment (start 27.5000 12.0000) (end 25.5000 10.0000) (width 0.180) (layer "B.Cu") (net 2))
 (segment (start 25.5000 10.0000) (end 23.5000 10.0000) (width 0.180) (layer "B.Cu") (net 2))
 (segment (start 23.5000 10.0000) (end 22.5000 9.0000) (width 0.180) (layer "B.Cu") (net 2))
 (segment (start 22.5000 9.0000) (end 21.5000 9.0000) (width 0.180) (layer "B.Cu") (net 2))
 (segment (start 21.5000 9.0000) (end 20.5000 10.0000) (width 0.180) (layer "B.Cu") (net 2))
 (segment (start 20.5000 10.0000) (end 17.5000 10.0000) (width 0.180) (layer "B.Cu") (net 2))
 (segment (start 17.5000 10.0000) (end 17.0000 10.0000) (width 0.180) (layer "F.Cu") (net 2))
 (segment (start 27.5000 12.0000) (end 22.0000 6.5000) (width 0.180) (layer "B.Cu") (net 2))
 (segment (start 22.0000 6.5000) (end 20.5000 6.5000) (width 0.180) (layer "B.Cu") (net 2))
 (via (at 22.5000 14.0000) (size 0.560) (drill 0.300) (layers "F.Cu" "B.Cu") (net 12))
 (via (at 28.5000 16.5000) (size 0.560) (drill 0.300) (layers "F.Cu" "B.Cu") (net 12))
 (via (at 4.5000 17.5000) (size 0.560) (drill 0.300) (layers "F.Cu" "B.Cu") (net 1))
 (via (at 18.5000 17.5000) (size 0.560) (drill 0.300) (layers "F.Cu" "B.Cu") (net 3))
 (via (at 24.5000 17.5000) (size 0.560) (drill 0.300) (layers "F.Cu" "B.Cu") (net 3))
 (via (at 7.0000 17.5000) (size 0.560) (drill 0.300) (layers "F.Cu" "B.Cu") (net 3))
 (via (at 13.5000 5.5000) (size 0.560) (drill 0.300) (layers "F.Cu" "B.Cu") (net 3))
 (via (at 25.0000 14.5000) (size 0.560) (drill 0.300) (layers "F.Cu" "B.Cu") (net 2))
 (via (at 27.0000 4.5000) (size 0.560) (drill 0.300) (layers "F.Cu" "B.Cu") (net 2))
 (via (at 16.5000 10.0000) (size 0.560) (drill 0.300) (layers "F.Cu" "B.Cu") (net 2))
 (via (at 16.5000 21.5000) (size 0.560) (drill 0.300) (layers "F.Cu" "B.Cu") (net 2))
 (via (at 11.0000 14.0000) (size 0.560) (drill 0.300) (layers "F.Cu" "B.Cu") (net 2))
 (via (at 17.5000 10.0000) (size 0.560) (drill 0.300) (layers "F.Cu" "B.Cu") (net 2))
 (via (at 20.5000 6.5000) (size 0.560) (drill 0.300) (layers "F.Cu" "B.Cu") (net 2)))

